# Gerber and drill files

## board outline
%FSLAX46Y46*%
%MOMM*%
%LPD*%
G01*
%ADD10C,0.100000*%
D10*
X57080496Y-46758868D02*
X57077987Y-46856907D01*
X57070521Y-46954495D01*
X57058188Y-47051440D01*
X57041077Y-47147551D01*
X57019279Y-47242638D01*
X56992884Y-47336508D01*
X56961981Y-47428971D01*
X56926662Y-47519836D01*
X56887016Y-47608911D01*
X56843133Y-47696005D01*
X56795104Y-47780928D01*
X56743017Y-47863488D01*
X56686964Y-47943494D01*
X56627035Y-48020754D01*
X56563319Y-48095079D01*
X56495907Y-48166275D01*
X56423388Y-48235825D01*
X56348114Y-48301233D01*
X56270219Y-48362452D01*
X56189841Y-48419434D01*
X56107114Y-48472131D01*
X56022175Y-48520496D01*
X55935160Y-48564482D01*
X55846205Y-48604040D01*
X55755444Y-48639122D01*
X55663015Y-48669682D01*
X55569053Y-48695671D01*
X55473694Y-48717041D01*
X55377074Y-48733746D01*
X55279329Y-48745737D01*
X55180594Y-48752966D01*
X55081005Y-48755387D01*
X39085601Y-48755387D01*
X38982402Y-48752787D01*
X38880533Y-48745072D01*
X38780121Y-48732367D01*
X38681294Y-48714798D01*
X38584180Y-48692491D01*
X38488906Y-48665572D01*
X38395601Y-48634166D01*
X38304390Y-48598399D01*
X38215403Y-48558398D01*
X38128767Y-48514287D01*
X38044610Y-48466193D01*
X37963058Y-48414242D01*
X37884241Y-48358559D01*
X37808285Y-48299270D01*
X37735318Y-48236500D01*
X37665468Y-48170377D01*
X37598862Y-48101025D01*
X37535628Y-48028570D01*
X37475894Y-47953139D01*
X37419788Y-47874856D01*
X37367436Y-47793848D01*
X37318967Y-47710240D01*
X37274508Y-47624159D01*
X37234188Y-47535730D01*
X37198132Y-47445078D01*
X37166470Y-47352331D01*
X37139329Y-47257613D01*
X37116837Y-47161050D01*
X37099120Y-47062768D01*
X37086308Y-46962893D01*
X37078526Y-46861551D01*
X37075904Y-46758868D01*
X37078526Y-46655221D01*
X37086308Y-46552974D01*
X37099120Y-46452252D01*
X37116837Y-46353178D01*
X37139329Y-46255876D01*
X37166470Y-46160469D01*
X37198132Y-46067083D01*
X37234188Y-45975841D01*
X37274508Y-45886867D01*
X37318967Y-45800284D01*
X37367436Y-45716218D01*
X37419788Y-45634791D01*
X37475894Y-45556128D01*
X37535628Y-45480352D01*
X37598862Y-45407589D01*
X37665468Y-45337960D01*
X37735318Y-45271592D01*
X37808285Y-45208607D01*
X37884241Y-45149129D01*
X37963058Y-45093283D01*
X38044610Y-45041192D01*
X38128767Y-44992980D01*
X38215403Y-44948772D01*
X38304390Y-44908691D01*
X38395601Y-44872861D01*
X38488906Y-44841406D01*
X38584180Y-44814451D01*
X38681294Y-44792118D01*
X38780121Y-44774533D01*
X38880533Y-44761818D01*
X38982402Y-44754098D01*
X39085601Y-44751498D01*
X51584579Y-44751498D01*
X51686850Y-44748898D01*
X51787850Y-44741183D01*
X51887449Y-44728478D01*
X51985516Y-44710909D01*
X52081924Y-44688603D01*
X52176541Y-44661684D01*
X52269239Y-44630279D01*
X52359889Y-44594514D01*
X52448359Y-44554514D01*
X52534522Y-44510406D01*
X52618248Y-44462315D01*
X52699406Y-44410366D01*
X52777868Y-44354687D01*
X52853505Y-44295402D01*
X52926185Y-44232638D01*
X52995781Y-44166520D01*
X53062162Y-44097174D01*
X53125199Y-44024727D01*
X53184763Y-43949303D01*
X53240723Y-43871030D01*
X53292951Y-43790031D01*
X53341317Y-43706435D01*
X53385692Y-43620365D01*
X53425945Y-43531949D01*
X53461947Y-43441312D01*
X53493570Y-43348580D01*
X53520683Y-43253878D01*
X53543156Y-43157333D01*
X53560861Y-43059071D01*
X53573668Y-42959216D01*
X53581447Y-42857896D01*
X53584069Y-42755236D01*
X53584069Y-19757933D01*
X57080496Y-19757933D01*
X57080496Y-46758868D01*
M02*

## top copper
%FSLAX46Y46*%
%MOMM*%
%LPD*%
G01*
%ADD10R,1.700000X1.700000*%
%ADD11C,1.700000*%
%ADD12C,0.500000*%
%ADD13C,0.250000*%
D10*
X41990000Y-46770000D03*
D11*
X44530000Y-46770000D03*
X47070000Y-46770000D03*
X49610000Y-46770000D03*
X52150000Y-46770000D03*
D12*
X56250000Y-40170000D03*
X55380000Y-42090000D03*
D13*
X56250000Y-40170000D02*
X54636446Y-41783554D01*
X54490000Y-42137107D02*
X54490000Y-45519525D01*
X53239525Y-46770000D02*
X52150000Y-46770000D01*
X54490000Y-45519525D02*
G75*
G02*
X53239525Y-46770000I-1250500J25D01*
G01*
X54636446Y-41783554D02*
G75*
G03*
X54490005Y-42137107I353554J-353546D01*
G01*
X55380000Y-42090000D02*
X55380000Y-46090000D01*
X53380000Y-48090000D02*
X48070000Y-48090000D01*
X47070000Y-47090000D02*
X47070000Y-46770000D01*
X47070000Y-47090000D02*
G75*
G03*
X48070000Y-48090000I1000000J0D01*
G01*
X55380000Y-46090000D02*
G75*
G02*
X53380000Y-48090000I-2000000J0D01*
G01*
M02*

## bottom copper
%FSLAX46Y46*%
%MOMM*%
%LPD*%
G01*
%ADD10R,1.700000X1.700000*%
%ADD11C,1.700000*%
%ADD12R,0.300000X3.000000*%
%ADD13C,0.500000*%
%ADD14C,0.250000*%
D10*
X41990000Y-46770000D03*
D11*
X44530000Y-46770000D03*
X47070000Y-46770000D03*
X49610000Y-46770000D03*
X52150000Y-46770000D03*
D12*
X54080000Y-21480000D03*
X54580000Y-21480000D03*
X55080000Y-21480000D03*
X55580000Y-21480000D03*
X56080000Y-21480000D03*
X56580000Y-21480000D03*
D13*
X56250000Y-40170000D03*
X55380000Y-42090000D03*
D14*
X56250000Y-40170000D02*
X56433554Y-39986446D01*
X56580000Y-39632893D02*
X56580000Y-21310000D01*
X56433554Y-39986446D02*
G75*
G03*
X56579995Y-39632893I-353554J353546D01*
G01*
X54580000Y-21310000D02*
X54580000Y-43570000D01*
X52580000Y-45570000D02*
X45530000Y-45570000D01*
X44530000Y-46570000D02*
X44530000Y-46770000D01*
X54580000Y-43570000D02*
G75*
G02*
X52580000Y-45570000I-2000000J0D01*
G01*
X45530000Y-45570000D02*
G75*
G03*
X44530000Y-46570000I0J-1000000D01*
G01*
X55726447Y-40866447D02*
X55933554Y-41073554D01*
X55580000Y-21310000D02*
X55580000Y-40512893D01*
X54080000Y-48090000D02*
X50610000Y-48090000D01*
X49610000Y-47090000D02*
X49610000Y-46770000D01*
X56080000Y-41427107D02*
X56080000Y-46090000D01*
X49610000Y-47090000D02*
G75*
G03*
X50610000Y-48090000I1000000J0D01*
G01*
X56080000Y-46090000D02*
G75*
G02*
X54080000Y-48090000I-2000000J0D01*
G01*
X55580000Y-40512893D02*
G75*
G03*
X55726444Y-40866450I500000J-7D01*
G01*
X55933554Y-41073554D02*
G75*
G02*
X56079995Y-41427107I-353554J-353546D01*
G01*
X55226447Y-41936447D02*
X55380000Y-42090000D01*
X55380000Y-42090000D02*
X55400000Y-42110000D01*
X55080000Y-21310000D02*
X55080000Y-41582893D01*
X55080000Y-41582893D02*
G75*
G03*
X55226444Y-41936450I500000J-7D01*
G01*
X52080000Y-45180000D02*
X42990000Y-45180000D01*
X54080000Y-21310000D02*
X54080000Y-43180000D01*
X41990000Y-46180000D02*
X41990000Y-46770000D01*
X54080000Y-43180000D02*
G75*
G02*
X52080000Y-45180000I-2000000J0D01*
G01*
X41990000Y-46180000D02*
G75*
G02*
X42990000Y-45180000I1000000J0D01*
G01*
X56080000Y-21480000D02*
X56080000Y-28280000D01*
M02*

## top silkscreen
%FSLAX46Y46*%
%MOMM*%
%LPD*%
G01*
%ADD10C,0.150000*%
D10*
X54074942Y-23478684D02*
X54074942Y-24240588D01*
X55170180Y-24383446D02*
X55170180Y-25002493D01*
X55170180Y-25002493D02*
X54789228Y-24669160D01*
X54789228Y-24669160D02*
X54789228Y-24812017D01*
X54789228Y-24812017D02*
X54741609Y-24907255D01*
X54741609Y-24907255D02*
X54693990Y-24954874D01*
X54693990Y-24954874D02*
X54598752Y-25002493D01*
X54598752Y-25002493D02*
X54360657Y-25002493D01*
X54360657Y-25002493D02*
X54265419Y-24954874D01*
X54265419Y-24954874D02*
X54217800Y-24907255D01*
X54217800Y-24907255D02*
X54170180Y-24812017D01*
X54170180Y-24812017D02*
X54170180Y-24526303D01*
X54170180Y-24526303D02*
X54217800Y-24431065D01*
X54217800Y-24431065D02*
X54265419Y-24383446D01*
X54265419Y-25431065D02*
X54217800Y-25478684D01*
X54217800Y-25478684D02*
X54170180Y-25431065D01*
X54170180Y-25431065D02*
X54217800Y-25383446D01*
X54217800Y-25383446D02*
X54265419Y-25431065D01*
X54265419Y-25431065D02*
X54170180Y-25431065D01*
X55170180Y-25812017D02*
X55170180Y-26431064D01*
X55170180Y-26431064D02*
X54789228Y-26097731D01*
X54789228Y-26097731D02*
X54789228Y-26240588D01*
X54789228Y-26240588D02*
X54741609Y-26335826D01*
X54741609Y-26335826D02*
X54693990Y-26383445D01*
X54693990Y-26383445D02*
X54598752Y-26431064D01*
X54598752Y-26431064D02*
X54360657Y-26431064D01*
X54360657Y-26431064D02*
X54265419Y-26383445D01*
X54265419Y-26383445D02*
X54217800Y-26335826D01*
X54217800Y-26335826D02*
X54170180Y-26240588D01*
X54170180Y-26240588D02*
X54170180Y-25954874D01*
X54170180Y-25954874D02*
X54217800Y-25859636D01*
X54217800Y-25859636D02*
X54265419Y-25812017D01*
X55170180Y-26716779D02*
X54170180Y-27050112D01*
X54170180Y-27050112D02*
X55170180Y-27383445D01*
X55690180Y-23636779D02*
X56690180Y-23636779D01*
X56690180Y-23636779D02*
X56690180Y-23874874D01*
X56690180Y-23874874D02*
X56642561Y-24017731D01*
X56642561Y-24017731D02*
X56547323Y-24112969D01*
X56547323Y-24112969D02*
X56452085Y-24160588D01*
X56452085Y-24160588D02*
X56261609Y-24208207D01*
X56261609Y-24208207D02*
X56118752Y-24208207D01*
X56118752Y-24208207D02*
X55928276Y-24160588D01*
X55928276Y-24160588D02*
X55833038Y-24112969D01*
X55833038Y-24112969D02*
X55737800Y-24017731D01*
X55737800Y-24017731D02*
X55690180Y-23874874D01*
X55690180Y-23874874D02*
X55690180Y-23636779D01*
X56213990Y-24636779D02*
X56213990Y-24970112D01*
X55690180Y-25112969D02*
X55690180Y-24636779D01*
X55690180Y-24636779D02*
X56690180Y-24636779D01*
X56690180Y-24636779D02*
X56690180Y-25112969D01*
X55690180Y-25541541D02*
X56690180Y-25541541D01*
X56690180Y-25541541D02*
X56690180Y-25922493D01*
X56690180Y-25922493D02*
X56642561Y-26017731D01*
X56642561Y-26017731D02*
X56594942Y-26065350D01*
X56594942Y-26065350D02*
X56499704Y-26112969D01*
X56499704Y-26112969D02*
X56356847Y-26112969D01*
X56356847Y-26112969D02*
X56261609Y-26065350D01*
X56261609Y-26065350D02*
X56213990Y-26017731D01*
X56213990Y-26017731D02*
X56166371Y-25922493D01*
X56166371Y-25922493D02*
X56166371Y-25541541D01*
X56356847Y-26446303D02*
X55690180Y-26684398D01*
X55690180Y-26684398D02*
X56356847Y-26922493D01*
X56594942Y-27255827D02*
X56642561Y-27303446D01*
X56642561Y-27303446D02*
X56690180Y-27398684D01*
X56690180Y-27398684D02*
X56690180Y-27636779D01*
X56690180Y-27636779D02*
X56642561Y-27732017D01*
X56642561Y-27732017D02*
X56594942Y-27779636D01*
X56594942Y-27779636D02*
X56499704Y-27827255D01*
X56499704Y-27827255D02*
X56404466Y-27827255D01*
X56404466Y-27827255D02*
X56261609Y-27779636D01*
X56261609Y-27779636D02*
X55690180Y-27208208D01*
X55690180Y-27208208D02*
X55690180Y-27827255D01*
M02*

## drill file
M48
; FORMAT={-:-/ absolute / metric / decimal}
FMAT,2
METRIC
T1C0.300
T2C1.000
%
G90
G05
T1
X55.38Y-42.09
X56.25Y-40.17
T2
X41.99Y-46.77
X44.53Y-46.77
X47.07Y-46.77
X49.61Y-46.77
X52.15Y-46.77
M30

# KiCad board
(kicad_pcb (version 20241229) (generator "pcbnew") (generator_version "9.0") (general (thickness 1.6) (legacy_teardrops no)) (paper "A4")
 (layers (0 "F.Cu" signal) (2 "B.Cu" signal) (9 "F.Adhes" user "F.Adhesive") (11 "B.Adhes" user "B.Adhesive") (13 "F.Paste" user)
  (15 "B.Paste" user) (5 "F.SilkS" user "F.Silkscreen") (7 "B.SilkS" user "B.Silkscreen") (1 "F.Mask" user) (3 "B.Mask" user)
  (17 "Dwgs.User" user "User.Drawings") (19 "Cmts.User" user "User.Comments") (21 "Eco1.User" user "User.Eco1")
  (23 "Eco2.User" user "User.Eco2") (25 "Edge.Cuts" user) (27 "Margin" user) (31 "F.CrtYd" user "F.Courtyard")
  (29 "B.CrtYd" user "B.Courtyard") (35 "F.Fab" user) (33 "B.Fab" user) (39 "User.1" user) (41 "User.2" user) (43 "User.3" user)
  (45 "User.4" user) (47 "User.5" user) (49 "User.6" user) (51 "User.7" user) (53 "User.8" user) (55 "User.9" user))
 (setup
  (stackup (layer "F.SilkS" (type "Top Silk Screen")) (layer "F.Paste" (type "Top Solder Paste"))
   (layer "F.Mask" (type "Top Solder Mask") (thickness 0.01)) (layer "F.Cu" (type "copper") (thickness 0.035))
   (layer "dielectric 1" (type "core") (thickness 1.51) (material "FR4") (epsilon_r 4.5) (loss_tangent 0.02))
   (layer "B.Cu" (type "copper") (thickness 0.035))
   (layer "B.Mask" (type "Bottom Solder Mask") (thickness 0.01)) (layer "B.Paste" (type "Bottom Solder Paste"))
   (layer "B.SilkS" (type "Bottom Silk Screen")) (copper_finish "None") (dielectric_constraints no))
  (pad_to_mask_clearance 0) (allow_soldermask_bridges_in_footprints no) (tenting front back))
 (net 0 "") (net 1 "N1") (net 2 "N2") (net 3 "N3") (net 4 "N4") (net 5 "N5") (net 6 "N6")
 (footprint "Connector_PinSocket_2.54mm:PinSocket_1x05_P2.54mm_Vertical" (layer "F.Cu") (at 41.99 46.77 90)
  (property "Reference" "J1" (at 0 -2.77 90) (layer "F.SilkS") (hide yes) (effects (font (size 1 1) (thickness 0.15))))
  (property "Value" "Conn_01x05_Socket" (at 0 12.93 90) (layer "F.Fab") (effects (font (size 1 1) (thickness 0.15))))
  (pad "1" thru_hole rect (at 0 0 90) (size 1.7 1.7) (drill 1) (layers "*.Cu" "*.Mask") (remove_unused_layers no) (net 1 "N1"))
  (pad "2" thru_hole circle (at 0 2.54 90) (size 1.7 1.7) (drill 1) (layers "*.Cu" "*.Mask") (remove_unused_layers no) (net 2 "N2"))
  (pad "3" thru_hole circle (at 0 5.08 90) (size 1.7 1.7) (drill 1) (layers "*.Cu" "*.Mask") (remove_unused_layers no) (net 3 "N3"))
  (pad "4" thru_hole circle (at 0 7.62 90) (size 1.7 1.7) (drill 1) (layers "*.Cu" "*.Mask") (remove_unused_layers no) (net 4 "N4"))
  (pad "5" thru_hole circle (at 0 10.16 90) (size 1.7 1.7) (drill 1) (layers "*.Cu" "*.Mask") (remove_unused_layers no) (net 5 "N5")))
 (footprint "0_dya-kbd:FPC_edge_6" (layer "B.Cu") (at 55.33 21.48)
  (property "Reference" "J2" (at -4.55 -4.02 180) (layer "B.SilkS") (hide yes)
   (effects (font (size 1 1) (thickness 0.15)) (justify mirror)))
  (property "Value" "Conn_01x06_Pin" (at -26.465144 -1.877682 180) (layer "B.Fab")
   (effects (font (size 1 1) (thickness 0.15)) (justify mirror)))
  (pad "1" smd rect (at -1.25 0) (size 0.3 3) (layers "B.Cu" "B.Mask" "B.Paste") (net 1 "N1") (thermal_bridge_angle 45))
  (pad "2" smd rect (at -0.75 0) (size 0.3 3) (layers "B.Cu" "B.Mask" "B.Paste") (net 2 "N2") (thermal_bridge_angle 45))
  (pad "3" smd rect (at -0.25 0) (size 0.3 3) (layers "B.Cu" "B.Mask" "B.Paste") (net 3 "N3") (thermal_bridge_angle 45))
  (pad "4" smd rect (at 0.25 0) (size 0.3 3) (layers "B.Cu" "B.Mask" "B.Paste") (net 4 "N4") (thermal_bridge_angle 45))
  (pad "5" smd rect (at 0.75 0) (size 0.3 3) (layers "B.Cu" "B.Mask" "B.Paste") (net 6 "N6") (thermal_bridge_angle 45))
  (pad "6" smd rect (at 1.25 0) (size 0.3 3) (layers "B.Cu" "B.Mask" "B.Paste") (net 5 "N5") (thermal_bridge_angle 45)))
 (gr_poly
  (pts (xy 57.080496 46.758868) (xy 57.077987 46.856907) (xy 57.070521 46.954495) (xy 57.058188 47.05144) (xy 57.041077 47.147551)
   (xy 57.019279 47.242638) (xy 56.992884 47.336508) (xy 56.961981 47.428971) (xy 56.926662 47.519836) (xy 56.887016 47.608911)
   (xy 56.843133 47.696005) (xy 56.795104 47.780928) (xy 56.743017 47.863488) (xy 56.686964 47.943494) (xy 56.627035 48.020754)
   (xy 56.563319 48.095079) (xy 56.495907 48.166275) (xy 56.423388 48.235825) (xy 56.348114 48.301233) (xy 56.270219 48.362452)
   (xy 56.189841 48.419434) (xy 56.107114 48.472131) (xy 56.022175 48.520496) (xy 55.93516 48.564482) (xy 55.846205 48.60404)
   (xy 55.755444 48.639122) (xy 55.663015 48.669682) (xy 55.569053 48.695671) (xy 55.473694 48.717041) (xy 55.377074 48.733746)
   (xy 55.279329 48.745737) (xy 55.180594 48.752966) (xy 55.081005 48.755387) (xy 39.085601 48.755387) (xy 38.982402 48.752787)
   (xy 38.880533 48.745072) (xy 38.780121 48.732367) (xy 38.681294 48.714798) (xy 38.58418 48.692491) (xy 38.488906 48.665572)
   (xy 38.395601 48.634166) (xy 38.30439 48.598399) (xy 38.215403 48.558398) (xy 38.128767 48.514287) (xy 38.04461 48.466193)
   (xy 37.963058 48.414242) (xy 37.884241 48.358559) (xy 37.808285 48.29927) (xy 37.735318 48.2365) (xy 37.665468 48.170377)
   (xy 37.598862 48.101025) (xy 37.535628 48.02857) (xy 37.475894 47.953139) (xy 37.419788 47.874856) (xy 37.367436 47.793848)
   (xy 37.318967 47.71024) (xy 37.274508 47.624159) (xy 37.234188 47.53573) (xy 37.198132 47.445078) (xy 37.16647 47.352331)
   (xy 37.139329 47.257613) (xy 37.116837 47.16105) (xy 37.09912 47.062768) (xy 37.086308 46.962893) (xy 37.078526 46.861551)
   (xy 37.075904 46.758868) (xy 37.078526 46.655221) (xy 37.086308 46.552974) (xy 37.09912 46.452252) (xy 37.116837 46.353178)
   (xy 37.139329 46.255876) (xy 37.16647 46.160469) (xy 37.198132 46.067083) (xy 37.234188 45.975841) (xy 37.274508 45.886867)
   (xy 37.318967 45.800284) (xy 37.367436 45.716218) (xy 37.419788 45.634791) (xy 37.475894 45.556128) (xy 37.535628 45.480352)
   (xy 37.598862 45.407589) (xy 37.665468 45.33796) (xy 37.735318 45.271592) (xy 37.808285 45.208607) (xy 37.884241 45.149129)
   (xy 37.963058 45.093283) (xy 38.04461 45.041192) (xy 38.128767 44.99298) (xy 38.215403 44.948772) (xy 38.30439 44.908691)
   (xy 38.395601 44.872861) (xy 38.488906 44.841406) (xy 38.58418 44.814451) (xy 38.681294 44.792118) (xy 38.780121 44.774533)
   (xy 38.880533 44.761818) (xy 38.982402 44.754098) (xy 39.085601 44.751498) (xy 51.584579 44.751498) (xy 51.68685 44.748898)
   (xy 51.78785 44.741183) (xy 51.887449 44.728478) (xy 51.985516 44.710909) (xy 52.081924 44.688603) (xy 52.176541 44.661684)
   (xy 52.269239 44.630279) (xy 52.359889 44.594514) (xy 52.448359 44.554514) (xy 52.534522 44.510406) (xy 52.618248 44.462315)
   (xy 52.699406 44.410366) (xy 52.777868 44.354687) (xy 52.853505 44.295402) (xy 52.926185 44.232638) (xy 52.995781 44.16652)
   (xy 53.062162 44.097174) (xy 53.125199 44.024727) (xy 53.184763 43.949303) (xy 53.240723 43.87103) (xy 53.292951 43.790031)
   (xy 53.341317 43.706435) (xy 53.385692 43.620365) (xy 53.425945 43.531949) (xy 53.461947 43.441312) (xy 53.49357 43.34858)
   (xy 53.520683 43.253878) (xy 53.543156 43.157333) (xy 53.560861 43.059071) (xy 53.573668 42.959216) (xy 53.581447 42.857896)
   (xy 53.584069 42.755236) (xy 53.584069 19.757933) (xy 57.080496 19.757933))
  (stroke (width 0.1) (type solid) (color 0 255 43 1)) (fill no) (layer "Edge.Cuts"))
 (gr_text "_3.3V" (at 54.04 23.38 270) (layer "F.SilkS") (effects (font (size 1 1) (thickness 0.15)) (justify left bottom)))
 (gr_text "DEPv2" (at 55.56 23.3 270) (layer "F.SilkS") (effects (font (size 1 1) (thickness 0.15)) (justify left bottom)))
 (segment (start 56.25 40.17) (end 54.636446 41.783554) (width 0.25) (layer "F.Cu") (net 5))
 (segment (start 54.49 42.137107) (end 54.49 45.519525) (width 0.25) (layer "F.Cu") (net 5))
 (segment (start 53.239525 46.77) (end 52.15 46.77) (width 0.25) (layer "F.Cu") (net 5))
 (via (at 56.25 40.17) (size 0.5) (drill 0.3) (layers "F.Cu" "B.Cu") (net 5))
 (arc (start 54.49 45.519525) (mid 54.123744 46.403744) (end 53.239525 46.77) (width 0.25) (layer "F.Cu") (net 5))
 (arc (start 54.636446 41.783554) (mid 54.52806 41.945766) (end 54.49 42.137107) (width 0.25) (layer "F.Cu") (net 5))
 (segment (start 56.25 40.17) (end 56.433554 39.986446) (width 0.25) (layer "B.Cu") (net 5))
 (segment (start 56.58 39.632893) (end 56.58 21.31) (width 0.25) (layer "B.Cu") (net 5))
 (arc (start 56.433554 39.986446) (mid 56.54194 39.824234) (end 56.58 39.632893) (width 0.25) (layer "B.Cu") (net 5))
 (segment (start 54.58 21.31) (end 54.58 43.57) (width 0.25) (layer "B.Cu") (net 2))
 (segment (start 52.58 45.57) (end 45.53 45.57) (width 0.25) (layer "B.Cu") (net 2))
 (segment (start 44.53 46.57) (end 44.53 46.77) (width 0.25) (layer "B.Cu") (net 2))
 (arc (start 54.58 43.57) (mid 53.994214 44.984214) (end 52.58 45.57) (width 0.25) (layer "B.Cu") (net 2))
 (arc (start 45.53 45.57) (mid 44.822893 45.862893) (end 44.53 46.57) (width 0.25) (layer "B.Cu") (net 2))
 (segment (start 55.726447 40.866447) (end 55.933554 41.073554) (width 0.25) (layer "B.Cu") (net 4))
 (segment (start 55.58 21.31) (end 55.58 40.512893) (width 0.25) (layer "B.Cu") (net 4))
 (segment (start 54.08 48.09) (end 50.61 48.09) (width 0.25) (layer "B.Cu") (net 4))
 (segment (start 49.61 47.09) (end 49.61 46.77) (width 0.25) (layer "B.Cu") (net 4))
 (segment (start 56.08 41.427107) (end 56.08 46.09) (width 0.25) (layer "B.Cu") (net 4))
 (arc (start 49.61 47.09) (mid 49.902893 47.797107) (end 50.61 48.09) (width 0.25) (layer "B.Cu") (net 4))
 (arc (start 56.08 46.09) (mid 55.494214 47.504214) (end 54.08 48.09) (width 0.25) (layer "B.Cu") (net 4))
 (arc (start 55.58 40.512893) (mid 55.61806 40.704235) (end 55.726447 40.866447) (width 0.25) (layer "B.Cu") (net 4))
 (arc (start 55.933554 41.073554) (mid 56.04194 41.235766) (end 56.08 41.427107) (width 0.25) (layer "B.Cu") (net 4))
 (segment (start 55.38 42.09) (end 55.38 46.09) (width 0.25) (layer "F.Cu") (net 3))
 (segment (start 53.38 48.09) (end 48.07 48.09) (width 0.25) (layer "F.Cu") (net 3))
 (segment (start 47.07 47.09) (end 47.07 46.77) (width 0.25) (layer "F.Cu") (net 3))
 (via (at 55.38 42.09) (size 0.5) (drill 0.3) (layers "F.Cu" "B.Cu") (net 3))
 (arc (start 47.07 47.09) (mid 47.362893 47.797107) (end 48.07 48.09) (width 0.25) (layer "F.Cu") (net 3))
 (arc (start 55.38 46.09) (mid 54.794214 47.504214) (end 53.38 48.09) (width 0.25) (layer "F.Cu") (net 3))
 (segment (start 55.226447 41.936447) (end 55.38 42.09) (width 0.25) (layer "B.Cu") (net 3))
 (segment (start 55.38 42.09) (end 55.4 42.11) (width 0.25) (layer "B.Cu") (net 3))
 (segment (start 55.08 21.31) (end 55.08 41.582893) (width 0.25) (layer "B.Cu") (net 3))
 (arc (start 55.08 41.582893) (mid 55.11806 41.774235) (end 55.226447 41.936447) (width 0.25) (layer "B.Cu") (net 3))
 (segment (start 52.08 45.18) (end 42.99 45.18) (width 0.25) (layer "B.Cu") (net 1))
 (segment (start 54.08 21.31) (end 54.08 43.18) (width 0.25) (layer "B.Cu") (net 1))
 (segment (start 41.99 46.18) (end 41.99 46.77) (width 0.25) (layer "B.Cu") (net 1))
 (arc (start 54.08 43.18) (mid 53.494214 44.594214) (end 52.08 45.18) (width 0.25) (layer "B.Cu") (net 1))
 (arc (start 41.99 46.18) (mid 42.282893 45.472893) (end 42.99 45.18) (width 0.25) (layer "B.Cu") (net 1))
 (segment (start 56.08 21.48) (end 56.08 28.28) (width 0.25) (layer "B.Cu") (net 6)))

